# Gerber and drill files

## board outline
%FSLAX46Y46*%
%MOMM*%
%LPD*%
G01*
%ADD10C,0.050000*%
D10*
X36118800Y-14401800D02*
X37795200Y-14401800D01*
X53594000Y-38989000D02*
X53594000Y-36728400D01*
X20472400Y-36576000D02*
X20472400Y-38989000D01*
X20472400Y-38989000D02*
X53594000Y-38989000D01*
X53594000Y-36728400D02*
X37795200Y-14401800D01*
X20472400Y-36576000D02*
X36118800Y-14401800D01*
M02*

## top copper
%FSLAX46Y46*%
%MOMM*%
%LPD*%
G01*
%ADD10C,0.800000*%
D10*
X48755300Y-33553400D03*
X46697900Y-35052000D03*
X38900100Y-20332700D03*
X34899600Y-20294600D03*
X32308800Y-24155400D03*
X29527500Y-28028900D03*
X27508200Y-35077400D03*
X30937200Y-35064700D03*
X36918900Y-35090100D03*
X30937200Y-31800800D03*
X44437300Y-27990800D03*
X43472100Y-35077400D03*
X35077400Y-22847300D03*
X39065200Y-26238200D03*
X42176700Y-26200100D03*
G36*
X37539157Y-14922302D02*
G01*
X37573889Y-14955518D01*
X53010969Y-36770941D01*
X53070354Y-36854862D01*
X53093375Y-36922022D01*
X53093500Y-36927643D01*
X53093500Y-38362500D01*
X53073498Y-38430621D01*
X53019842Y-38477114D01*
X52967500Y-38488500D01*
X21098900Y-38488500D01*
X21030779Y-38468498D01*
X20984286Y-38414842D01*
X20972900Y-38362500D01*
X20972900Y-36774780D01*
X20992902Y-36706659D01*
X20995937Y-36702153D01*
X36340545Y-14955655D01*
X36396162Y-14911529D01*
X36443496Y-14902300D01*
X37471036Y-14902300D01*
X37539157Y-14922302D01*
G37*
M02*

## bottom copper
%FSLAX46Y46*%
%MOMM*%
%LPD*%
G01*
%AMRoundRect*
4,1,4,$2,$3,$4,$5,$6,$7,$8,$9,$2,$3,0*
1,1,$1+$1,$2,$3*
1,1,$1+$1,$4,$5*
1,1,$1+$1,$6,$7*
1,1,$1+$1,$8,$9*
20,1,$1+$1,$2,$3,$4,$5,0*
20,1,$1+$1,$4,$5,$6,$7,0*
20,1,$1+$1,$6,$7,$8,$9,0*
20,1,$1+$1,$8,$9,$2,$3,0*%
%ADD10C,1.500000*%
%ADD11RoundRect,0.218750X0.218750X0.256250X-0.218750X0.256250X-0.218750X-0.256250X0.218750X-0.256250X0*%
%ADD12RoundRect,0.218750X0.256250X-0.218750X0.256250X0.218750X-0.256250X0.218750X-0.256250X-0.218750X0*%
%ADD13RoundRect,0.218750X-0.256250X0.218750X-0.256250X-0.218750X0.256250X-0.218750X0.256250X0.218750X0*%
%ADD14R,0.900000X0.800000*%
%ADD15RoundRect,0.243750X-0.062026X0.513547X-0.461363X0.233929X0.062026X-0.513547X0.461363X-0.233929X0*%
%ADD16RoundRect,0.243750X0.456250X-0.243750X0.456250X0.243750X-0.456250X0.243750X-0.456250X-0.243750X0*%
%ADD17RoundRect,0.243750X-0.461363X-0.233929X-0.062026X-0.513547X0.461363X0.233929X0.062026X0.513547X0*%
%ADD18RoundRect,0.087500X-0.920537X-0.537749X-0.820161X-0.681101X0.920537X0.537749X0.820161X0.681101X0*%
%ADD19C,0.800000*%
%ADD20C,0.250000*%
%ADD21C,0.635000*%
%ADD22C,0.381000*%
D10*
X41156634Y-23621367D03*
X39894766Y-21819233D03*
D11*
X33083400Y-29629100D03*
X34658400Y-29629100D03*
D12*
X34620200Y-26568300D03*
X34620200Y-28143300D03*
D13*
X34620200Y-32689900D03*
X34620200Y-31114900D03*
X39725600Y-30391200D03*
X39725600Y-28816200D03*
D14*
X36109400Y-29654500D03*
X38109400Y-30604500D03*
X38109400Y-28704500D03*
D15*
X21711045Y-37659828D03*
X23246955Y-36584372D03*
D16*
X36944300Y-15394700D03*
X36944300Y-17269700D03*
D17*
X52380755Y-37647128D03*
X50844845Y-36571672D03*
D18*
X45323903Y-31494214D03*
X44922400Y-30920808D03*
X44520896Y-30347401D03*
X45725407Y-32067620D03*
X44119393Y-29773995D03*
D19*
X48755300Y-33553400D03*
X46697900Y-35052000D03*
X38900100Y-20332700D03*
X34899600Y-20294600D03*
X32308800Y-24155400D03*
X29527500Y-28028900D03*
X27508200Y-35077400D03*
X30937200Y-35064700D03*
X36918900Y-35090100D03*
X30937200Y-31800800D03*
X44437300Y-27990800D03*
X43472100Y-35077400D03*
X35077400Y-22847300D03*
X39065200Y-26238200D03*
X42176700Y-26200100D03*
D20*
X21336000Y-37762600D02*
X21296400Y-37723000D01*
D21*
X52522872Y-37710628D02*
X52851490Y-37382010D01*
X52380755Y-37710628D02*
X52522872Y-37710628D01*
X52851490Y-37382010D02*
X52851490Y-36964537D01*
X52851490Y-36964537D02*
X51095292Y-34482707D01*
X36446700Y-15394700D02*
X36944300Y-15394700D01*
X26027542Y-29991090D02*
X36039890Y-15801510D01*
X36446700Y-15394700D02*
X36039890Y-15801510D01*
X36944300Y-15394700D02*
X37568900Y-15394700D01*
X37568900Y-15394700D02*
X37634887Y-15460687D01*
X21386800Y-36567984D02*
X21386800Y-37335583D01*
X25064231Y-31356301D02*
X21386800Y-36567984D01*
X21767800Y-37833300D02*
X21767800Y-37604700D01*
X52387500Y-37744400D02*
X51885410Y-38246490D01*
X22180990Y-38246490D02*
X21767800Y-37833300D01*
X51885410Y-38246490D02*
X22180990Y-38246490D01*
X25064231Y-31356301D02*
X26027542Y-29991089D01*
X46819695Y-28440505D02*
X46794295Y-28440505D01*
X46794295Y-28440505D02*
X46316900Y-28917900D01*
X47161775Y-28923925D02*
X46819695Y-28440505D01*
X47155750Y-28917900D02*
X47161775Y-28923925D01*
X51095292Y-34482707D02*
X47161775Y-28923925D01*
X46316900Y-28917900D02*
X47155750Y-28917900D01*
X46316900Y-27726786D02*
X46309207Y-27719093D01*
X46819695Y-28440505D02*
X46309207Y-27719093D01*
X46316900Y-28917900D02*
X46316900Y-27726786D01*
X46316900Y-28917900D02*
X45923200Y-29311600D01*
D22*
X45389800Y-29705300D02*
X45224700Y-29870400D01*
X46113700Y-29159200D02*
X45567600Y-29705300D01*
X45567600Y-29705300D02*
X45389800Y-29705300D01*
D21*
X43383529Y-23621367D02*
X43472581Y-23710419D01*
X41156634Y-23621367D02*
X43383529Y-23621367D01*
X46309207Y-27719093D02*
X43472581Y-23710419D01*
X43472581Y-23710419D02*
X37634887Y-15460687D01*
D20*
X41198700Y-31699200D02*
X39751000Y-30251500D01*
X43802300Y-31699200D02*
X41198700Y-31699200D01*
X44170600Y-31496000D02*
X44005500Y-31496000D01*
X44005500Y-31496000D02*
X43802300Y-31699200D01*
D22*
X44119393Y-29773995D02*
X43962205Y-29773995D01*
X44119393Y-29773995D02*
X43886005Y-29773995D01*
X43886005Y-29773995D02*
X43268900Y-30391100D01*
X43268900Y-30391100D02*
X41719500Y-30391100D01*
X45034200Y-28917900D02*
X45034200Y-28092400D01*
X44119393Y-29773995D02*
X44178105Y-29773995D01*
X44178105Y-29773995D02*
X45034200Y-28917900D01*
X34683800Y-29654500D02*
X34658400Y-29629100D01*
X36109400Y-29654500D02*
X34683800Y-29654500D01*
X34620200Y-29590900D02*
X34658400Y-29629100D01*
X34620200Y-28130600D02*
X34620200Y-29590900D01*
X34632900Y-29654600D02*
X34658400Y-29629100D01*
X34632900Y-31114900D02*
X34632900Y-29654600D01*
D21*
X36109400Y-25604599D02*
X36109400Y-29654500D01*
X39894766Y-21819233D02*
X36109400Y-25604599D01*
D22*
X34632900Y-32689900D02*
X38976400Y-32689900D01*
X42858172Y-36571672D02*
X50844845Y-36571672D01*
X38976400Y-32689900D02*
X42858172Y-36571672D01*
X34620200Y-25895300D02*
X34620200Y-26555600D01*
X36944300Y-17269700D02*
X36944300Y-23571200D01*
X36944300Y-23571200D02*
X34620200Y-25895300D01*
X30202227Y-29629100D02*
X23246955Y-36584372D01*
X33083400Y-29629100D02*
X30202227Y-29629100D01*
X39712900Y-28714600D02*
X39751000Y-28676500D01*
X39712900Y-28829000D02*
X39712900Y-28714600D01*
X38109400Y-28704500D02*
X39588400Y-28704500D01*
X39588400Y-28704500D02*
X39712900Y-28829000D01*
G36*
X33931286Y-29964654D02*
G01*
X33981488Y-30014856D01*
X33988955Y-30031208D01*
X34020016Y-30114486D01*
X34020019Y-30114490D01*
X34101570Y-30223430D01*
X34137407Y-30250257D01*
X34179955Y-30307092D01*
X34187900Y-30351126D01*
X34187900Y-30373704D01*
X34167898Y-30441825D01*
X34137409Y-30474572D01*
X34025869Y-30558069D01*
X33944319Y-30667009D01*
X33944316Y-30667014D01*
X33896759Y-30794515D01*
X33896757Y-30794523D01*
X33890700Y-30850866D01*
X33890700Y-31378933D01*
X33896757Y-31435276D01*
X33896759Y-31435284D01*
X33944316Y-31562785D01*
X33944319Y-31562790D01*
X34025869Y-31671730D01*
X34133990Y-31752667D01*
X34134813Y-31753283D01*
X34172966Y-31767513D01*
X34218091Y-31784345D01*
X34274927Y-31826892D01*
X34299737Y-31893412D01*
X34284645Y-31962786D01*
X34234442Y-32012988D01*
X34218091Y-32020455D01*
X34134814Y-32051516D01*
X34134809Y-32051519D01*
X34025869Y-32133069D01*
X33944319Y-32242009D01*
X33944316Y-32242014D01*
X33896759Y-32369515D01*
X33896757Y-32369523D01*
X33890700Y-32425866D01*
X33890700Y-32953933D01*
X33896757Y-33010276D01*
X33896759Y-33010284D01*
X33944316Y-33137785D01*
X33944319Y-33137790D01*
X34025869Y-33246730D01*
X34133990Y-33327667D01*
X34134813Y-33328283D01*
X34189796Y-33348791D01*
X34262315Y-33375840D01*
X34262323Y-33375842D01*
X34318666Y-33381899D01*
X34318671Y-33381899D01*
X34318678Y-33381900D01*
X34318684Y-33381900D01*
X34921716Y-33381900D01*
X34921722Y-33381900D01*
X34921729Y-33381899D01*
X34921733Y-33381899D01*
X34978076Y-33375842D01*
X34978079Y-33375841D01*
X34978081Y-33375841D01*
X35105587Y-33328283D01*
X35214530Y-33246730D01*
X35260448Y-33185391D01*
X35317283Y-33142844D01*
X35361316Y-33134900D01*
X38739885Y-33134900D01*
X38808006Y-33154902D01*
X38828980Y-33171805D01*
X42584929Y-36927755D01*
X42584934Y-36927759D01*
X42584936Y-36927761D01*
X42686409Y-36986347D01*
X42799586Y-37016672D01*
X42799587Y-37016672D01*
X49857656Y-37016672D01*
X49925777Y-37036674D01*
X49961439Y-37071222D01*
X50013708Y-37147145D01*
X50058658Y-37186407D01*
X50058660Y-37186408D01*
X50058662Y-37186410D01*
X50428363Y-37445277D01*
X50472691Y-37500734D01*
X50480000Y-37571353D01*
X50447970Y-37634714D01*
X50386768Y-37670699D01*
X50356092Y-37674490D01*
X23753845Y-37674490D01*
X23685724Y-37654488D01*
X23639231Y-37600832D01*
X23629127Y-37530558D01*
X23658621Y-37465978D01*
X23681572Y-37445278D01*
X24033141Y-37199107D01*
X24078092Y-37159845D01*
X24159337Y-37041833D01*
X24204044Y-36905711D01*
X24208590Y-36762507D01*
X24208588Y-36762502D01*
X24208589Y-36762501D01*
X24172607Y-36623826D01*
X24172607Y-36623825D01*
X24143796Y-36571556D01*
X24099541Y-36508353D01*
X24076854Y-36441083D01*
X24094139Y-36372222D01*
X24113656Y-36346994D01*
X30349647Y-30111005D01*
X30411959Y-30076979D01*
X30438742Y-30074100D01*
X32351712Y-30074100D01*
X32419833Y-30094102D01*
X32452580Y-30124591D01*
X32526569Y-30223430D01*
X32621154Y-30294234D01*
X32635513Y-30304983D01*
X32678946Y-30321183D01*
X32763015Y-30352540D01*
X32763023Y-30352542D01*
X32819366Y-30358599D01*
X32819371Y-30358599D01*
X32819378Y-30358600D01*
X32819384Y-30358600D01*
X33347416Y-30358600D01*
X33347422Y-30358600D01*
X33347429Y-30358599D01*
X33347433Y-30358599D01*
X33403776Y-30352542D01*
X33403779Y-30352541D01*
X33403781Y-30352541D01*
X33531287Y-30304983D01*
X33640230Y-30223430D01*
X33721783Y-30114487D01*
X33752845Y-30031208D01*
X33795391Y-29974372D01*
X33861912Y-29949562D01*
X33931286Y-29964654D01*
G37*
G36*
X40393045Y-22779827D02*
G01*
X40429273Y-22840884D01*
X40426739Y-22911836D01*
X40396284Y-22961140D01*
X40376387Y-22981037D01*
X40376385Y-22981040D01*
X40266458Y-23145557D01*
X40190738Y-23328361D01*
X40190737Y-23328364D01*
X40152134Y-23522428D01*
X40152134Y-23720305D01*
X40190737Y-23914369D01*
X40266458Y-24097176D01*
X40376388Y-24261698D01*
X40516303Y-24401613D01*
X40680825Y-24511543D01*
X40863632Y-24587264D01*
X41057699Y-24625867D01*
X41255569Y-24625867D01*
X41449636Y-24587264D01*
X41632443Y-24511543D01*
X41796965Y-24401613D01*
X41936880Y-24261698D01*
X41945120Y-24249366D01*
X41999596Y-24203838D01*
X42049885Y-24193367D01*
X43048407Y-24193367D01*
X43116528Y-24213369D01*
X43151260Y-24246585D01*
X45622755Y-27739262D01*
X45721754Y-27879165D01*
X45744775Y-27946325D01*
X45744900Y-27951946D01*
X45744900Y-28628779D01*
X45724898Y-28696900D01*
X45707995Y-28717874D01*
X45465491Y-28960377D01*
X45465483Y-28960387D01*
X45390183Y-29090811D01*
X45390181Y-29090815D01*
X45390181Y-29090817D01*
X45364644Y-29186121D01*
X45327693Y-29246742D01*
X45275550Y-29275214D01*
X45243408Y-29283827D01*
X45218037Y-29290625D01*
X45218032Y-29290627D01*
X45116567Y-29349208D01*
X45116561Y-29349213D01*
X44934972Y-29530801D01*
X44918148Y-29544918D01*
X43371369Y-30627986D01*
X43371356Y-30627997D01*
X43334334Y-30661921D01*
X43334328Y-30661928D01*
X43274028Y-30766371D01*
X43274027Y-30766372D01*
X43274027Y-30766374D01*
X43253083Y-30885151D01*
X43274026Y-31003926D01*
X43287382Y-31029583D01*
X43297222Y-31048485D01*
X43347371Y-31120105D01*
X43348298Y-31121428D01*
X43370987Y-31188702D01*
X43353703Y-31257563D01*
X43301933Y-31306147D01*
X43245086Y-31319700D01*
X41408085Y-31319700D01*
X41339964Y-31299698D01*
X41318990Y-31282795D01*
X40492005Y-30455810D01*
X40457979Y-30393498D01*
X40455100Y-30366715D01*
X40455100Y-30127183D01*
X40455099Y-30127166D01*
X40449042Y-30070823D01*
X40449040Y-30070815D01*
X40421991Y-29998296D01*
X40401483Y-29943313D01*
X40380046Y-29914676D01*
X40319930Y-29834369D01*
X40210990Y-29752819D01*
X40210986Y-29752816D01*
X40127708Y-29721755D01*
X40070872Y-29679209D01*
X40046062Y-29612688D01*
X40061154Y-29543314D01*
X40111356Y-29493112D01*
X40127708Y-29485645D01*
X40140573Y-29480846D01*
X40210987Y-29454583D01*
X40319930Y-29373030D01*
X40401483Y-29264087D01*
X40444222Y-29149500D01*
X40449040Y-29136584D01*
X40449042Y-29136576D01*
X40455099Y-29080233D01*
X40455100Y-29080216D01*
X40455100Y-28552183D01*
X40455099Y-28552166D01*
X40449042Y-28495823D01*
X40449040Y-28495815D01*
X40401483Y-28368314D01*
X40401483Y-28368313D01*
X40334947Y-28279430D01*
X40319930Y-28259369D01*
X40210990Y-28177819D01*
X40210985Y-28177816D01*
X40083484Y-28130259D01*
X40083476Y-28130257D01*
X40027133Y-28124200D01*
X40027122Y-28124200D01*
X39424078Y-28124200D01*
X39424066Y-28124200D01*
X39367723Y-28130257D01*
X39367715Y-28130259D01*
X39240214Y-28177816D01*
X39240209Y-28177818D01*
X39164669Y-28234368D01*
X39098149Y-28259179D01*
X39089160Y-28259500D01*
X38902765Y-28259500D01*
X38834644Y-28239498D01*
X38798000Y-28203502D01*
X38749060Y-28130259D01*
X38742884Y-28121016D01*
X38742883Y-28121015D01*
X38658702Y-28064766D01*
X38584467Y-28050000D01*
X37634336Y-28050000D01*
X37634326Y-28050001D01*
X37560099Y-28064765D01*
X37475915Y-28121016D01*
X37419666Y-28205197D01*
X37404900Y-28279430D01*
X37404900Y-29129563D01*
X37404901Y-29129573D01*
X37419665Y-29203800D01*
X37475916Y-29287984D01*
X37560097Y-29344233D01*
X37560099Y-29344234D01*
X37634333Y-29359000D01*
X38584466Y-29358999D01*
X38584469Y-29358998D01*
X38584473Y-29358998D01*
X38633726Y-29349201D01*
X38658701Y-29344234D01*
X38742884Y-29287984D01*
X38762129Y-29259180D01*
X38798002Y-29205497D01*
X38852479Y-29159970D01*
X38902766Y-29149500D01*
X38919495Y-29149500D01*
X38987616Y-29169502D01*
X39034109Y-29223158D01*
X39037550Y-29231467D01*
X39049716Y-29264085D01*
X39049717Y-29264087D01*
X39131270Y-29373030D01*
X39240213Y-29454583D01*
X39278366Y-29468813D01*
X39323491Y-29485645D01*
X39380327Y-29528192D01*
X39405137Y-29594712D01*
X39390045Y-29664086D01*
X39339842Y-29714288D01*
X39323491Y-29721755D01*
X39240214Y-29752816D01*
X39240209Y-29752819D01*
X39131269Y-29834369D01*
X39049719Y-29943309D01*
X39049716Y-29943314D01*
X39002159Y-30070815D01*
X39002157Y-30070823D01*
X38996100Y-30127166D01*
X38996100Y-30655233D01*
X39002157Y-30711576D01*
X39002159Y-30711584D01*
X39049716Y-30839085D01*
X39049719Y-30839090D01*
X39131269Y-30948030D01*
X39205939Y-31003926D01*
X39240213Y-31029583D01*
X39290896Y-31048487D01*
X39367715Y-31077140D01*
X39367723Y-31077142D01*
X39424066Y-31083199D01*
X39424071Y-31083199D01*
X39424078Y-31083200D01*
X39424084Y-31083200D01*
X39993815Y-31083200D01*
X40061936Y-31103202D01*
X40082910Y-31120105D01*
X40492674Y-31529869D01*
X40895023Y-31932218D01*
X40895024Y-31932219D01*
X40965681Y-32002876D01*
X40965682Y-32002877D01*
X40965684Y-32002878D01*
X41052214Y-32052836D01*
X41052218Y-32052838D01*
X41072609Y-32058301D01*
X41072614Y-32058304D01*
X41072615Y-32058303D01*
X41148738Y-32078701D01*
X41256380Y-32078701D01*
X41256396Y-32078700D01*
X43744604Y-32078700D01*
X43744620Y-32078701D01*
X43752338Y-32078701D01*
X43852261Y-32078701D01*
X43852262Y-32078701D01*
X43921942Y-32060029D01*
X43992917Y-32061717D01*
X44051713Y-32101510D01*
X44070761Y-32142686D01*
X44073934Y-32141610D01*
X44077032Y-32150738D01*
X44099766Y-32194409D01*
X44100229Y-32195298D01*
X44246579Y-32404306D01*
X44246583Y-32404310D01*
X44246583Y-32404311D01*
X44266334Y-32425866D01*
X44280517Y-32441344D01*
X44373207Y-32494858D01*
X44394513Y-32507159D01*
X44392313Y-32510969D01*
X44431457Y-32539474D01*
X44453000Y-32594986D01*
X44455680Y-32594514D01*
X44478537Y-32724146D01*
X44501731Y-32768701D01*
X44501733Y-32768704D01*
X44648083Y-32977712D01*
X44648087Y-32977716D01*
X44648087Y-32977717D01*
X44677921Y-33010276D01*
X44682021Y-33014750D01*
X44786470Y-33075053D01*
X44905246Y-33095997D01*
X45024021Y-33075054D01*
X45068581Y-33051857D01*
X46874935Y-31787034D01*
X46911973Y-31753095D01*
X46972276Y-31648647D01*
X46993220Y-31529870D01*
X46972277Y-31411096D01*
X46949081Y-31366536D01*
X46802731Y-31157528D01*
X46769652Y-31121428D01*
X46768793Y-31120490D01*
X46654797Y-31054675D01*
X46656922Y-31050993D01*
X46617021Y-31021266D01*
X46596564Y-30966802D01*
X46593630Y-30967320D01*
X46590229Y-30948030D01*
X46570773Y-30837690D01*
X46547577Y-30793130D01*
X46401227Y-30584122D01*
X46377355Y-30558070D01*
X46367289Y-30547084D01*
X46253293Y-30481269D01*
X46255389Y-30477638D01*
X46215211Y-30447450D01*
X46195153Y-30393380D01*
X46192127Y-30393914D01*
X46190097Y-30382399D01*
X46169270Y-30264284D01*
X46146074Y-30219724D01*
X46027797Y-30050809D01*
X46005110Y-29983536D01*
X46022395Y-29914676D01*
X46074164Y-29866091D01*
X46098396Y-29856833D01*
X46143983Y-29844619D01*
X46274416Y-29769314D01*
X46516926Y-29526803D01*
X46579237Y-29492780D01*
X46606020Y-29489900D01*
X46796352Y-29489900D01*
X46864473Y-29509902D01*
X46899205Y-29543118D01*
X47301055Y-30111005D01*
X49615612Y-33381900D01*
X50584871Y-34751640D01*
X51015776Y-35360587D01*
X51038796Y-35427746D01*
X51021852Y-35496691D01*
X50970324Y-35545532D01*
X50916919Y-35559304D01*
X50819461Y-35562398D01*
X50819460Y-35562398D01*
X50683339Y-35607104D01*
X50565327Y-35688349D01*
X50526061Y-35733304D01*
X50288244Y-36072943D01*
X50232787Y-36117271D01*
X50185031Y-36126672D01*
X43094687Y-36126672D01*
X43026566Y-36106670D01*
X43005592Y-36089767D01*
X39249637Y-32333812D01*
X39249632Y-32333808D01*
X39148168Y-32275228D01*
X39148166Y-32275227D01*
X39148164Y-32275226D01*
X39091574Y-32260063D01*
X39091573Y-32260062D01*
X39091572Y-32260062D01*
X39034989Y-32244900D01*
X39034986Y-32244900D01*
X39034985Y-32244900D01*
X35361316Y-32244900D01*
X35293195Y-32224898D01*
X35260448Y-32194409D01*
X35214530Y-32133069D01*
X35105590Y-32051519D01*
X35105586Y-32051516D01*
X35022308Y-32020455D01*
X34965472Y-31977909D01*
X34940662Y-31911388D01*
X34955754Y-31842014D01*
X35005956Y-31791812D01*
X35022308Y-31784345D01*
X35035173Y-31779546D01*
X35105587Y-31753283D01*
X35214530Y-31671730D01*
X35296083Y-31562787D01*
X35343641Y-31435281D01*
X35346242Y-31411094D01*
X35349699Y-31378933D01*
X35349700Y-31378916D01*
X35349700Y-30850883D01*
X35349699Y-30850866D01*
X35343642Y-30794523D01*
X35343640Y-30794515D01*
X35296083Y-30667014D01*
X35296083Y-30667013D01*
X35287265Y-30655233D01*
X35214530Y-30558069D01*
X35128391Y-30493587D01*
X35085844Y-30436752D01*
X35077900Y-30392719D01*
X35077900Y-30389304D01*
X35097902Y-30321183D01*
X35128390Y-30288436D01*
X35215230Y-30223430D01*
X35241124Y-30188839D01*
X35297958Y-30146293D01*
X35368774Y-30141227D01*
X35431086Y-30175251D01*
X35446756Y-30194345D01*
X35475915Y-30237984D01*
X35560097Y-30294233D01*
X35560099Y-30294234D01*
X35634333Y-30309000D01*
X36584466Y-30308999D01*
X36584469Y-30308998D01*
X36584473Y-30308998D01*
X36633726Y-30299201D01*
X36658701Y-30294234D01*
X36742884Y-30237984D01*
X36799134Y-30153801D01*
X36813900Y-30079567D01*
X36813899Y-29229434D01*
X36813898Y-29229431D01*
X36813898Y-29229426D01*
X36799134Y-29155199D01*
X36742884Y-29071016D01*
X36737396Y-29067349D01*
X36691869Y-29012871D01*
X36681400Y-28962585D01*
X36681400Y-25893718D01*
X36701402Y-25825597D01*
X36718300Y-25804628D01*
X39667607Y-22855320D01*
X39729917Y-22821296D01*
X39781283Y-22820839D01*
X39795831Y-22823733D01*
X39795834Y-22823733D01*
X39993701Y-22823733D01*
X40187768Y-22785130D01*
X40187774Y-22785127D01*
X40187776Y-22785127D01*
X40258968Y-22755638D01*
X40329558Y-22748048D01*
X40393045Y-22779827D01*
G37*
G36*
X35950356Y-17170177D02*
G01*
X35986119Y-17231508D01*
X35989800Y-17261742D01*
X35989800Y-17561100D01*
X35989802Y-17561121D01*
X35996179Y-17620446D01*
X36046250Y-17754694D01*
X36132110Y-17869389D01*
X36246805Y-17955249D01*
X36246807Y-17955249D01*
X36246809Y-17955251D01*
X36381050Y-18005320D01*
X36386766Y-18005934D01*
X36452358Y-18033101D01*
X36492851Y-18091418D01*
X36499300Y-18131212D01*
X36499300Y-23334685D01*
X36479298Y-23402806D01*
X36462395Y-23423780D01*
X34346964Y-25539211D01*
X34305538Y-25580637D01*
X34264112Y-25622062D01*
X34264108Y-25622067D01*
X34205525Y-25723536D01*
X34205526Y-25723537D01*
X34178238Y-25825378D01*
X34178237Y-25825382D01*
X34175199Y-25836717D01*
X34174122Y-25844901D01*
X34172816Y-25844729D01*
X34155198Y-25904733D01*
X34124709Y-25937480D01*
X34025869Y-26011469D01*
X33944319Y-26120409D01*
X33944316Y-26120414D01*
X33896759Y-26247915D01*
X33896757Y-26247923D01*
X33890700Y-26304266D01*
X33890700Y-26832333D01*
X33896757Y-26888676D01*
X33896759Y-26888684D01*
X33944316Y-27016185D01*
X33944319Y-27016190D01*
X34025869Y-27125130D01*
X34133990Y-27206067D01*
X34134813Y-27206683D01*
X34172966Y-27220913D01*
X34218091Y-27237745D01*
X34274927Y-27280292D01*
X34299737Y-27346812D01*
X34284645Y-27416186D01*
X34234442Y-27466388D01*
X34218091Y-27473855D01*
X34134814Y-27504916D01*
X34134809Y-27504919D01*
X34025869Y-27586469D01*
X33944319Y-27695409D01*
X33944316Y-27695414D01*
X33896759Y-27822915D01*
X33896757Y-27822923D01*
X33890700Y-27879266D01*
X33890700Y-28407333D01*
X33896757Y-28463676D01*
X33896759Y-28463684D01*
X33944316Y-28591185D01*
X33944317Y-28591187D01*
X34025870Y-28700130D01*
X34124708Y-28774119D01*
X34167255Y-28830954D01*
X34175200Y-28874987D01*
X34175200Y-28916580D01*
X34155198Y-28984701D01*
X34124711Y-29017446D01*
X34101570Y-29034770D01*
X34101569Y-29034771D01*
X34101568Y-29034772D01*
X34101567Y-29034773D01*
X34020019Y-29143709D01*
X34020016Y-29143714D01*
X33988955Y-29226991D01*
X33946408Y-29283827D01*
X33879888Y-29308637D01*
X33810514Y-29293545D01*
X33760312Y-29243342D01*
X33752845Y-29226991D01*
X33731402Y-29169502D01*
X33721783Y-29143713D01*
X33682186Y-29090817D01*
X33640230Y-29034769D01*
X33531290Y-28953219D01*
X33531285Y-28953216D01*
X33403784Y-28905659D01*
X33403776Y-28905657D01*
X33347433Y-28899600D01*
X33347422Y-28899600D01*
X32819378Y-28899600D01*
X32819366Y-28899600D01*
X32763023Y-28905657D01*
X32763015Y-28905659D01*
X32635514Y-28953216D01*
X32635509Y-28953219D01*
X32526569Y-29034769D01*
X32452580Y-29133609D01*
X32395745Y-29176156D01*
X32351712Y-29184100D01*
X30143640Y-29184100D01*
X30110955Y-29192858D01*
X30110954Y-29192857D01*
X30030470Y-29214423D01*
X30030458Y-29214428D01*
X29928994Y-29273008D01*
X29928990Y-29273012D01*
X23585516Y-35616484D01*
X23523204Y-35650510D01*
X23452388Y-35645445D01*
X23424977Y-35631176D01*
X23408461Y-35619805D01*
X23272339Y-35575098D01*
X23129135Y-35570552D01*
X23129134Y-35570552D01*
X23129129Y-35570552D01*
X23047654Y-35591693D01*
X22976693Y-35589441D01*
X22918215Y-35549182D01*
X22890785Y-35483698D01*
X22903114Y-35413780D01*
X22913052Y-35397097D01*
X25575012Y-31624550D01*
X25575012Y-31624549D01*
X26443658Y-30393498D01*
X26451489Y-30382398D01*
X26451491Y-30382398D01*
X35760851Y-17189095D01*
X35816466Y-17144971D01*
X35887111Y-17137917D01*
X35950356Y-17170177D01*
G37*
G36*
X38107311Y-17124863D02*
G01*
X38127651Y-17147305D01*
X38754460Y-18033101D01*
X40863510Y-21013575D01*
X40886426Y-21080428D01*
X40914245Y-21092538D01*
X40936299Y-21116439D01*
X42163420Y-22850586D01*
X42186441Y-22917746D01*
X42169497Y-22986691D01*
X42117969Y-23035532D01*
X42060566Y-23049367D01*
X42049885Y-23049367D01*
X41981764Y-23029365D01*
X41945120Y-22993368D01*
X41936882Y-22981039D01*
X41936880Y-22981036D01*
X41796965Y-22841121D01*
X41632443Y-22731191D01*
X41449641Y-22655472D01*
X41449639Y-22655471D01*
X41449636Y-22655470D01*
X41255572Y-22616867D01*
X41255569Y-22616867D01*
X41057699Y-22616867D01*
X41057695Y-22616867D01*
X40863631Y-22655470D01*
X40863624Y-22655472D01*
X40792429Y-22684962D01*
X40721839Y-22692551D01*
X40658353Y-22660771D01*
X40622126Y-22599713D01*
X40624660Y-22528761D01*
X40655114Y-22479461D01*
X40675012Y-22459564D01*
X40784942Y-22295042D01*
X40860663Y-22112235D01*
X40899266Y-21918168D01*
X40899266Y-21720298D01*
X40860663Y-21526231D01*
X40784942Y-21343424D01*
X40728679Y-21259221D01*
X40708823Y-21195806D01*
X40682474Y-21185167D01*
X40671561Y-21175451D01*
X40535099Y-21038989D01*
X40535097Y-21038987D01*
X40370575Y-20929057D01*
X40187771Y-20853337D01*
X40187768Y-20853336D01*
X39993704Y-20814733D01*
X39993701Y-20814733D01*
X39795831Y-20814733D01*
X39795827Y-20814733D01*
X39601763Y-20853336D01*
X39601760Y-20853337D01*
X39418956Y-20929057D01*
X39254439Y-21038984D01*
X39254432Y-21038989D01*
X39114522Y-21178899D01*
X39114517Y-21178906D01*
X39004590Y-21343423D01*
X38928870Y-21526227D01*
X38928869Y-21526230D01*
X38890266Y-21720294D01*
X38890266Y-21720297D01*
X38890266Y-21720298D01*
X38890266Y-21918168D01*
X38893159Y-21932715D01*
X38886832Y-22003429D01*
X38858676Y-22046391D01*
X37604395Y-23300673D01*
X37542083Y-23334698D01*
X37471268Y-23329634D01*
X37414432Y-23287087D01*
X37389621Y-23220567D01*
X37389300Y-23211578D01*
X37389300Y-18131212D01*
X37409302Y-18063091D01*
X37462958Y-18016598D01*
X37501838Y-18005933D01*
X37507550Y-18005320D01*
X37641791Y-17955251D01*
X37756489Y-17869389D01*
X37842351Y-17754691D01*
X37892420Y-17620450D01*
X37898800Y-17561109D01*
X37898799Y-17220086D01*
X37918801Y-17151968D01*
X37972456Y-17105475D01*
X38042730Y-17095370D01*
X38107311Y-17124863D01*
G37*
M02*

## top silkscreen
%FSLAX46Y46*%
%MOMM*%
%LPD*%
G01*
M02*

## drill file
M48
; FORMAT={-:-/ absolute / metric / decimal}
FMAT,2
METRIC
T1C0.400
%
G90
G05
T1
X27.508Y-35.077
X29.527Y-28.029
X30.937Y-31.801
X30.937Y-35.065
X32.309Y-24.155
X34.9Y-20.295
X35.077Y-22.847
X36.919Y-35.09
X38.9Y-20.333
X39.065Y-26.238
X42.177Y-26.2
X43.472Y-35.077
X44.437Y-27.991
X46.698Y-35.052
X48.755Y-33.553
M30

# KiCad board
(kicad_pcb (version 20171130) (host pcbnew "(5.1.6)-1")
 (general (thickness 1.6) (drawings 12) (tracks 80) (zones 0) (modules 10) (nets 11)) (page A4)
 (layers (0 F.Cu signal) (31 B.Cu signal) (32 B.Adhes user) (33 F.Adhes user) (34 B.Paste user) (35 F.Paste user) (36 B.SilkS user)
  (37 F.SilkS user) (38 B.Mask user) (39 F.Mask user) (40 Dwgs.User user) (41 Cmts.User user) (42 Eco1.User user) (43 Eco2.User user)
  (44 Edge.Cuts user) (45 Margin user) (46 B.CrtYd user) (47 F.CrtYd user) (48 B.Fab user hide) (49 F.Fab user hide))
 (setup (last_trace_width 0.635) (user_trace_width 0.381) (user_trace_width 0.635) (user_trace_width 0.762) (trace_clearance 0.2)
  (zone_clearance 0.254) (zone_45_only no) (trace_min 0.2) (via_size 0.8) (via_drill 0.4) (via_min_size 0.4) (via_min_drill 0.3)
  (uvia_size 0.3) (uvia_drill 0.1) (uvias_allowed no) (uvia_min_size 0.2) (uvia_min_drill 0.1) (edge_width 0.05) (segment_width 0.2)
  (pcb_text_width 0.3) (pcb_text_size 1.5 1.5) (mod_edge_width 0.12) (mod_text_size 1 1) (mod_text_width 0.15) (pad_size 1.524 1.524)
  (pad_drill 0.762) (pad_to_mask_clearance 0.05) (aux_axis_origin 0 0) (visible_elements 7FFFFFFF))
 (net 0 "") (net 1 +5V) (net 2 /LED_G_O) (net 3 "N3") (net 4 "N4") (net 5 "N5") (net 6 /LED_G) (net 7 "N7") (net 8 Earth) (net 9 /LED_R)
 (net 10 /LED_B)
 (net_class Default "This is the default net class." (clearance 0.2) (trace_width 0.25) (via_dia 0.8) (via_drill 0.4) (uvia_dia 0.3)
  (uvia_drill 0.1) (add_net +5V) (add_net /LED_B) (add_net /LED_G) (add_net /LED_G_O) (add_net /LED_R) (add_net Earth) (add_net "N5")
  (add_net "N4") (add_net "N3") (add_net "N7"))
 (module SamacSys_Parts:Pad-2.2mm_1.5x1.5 (layer B.Cu) (at 40.5257 22.7203 125)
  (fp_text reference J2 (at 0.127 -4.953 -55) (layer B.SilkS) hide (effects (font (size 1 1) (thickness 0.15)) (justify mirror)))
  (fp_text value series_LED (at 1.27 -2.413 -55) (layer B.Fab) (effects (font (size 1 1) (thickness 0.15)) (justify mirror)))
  (pad 1 smd circle (at -1.1 0 125) (size 1.5 1.5) (layers B.Cu B.Paste B.Mask) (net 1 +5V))
  (pad 2 smd circle (at 1.1 0 125) (size 1.5 1.5) (layers B.Cu B.Paste B.Mask) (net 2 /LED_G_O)))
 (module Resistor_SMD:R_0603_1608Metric (layer B.Cu) (at 33.8709 29.6291 180)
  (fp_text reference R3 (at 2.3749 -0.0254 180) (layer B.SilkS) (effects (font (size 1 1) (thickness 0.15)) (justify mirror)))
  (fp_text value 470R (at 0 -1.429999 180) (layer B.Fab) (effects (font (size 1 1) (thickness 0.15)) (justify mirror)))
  (pad 2 smd roundrect (at 0.7875 0 180) (size 0.875 0.95) (layers B.Cu B.Paste B.Mask) (roundrect_rratio 0.25) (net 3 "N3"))
  (pad 1 smd roundrect (at -0.7875 0 180) (size 0.875 0.95) (layers B.Cu B.Paste B.Mask) (roundrect_rratio 0.25) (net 2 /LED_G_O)))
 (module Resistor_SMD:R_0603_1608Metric (layer B.Cu) (at 34.6202 27.3558 90)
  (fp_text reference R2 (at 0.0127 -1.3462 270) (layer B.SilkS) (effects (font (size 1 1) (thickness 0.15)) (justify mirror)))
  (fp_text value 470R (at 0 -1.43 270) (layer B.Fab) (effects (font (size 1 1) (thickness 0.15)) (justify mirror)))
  (pad 2 smd roundrect (at 0.7875 0 90) (size 0.875 0.95) (layers B.Cu B.Paste B.Mask) (roundrect_rratio 0.25) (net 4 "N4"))
  (pad 1 smd roundrect (at -0.7875 0 90) (size 0.875 0.95) (layers B.Cu B.Paste B.Mask) (roundrect_rratio 0.25) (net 2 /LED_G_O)))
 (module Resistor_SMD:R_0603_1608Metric (layer B.Cu) (at 34.6202 31.9024 270)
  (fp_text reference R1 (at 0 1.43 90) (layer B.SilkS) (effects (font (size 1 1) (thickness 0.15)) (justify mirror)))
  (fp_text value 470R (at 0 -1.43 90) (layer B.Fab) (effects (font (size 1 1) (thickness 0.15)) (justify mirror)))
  (pad 2 smd roundrect (at 0.7875 0 270) (size 0.875 0.95) (layers B.Cu B.Paste B.Mask) (roundrect_rratio 0.25) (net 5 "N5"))
  (pad 1 smd roundrect (at -0.7875 0 270) (size 0.875 0.95) (layers B.Cu B.Paste B.Mask) (roundrect_rratio 0.25) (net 2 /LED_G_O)))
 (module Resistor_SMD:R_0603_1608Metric (layer B.Cu) (at 39.7256 29.6037 270)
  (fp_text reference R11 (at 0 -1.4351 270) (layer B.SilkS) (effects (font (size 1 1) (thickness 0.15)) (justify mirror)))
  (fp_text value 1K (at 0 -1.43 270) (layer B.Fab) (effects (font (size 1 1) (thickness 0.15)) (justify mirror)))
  (pad 2 smd roundrect (at 0.7875 0 270) (size 0.875 0.95) (layers B.Cu B.Paste B.Mask) (roundrect_rratio 0.25) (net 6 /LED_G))
  (pad 1 smd roundrect (at -0.7875 0 270) (size 0.875 0.95) (layers B.Cu B.Paste B.Mask) (roundrect_rratio 0.25) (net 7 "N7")))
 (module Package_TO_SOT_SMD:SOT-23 (layer B.Cu) (at 37.1094 29.6545 180)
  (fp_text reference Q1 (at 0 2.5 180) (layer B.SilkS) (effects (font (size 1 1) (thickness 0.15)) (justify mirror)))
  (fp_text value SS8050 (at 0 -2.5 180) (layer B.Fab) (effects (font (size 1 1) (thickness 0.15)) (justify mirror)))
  (pad 3 smd rect (at 1 0 180) (size 0.9 0.8) (layers B.Cu B.Paste B.Mask) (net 2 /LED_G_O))
  (pad 2 smd rect (at -1 -0.95 180) (size 0.9 0.8) (layers B.Cu B.Paste B.Mask) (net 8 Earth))
  (pad 1 smd rect (at -1 0.95 180) (size 0.9 0.8) (layers B.Cu B.Paste B.Mask) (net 7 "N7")))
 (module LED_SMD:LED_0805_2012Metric (layer B.Cu) (at 22.479 37.1221 215)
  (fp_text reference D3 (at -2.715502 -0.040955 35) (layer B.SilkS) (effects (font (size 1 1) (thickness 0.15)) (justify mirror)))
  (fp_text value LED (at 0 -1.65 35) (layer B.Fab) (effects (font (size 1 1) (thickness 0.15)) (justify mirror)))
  (pad 2 smd roundrect (at 0.9375 0 215) (size 0.975 1.4) (layers B.Cu B.Paste B.Mask) (roundrect_rratio 0.25) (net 1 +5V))
  (pad 1 smd roundrect (at -0.9375 0 215) (size 0.975 1.4) (layers B.Cu B.Paste B.Mask) (roundrect_rratio 0.25) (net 3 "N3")))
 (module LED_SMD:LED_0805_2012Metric (layer B.Cu) (at 36.9443 16.3322 90)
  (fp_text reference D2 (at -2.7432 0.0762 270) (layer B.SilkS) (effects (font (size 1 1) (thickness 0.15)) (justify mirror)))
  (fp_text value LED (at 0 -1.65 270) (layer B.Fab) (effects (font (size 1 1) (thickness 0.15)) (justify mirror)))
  (pad 2 smd roundrect (at 0.9375 0 90) (size 0.975 1.4) (layers B.Cu B.Paste B.Mask) (roundrect_rratio 0.25) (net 1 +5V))
  (pad 1 smd roundrect (at -0.9375 0 90) (size 0.975 1.4) (layers B.Cu B.Paste B.Mask) (roundrect_rratio 0.25) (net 4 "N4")))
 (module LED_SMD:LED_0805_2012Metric (layer B.Cu) (at 51.6128 37.1094 325)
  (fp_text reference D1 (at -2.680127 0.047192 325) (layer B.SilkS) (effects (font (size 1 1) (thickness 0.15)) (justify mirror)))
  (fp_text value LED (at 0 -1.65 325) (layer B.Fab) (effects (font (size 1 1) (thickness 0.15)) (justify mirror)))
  (pad 2 smd roundrect (at 0.9375 0 325) (size 0.975 1.4) (layers B.Cu B.Paste B.Mask) (roundrect_rratio 0.25) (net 1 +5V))
  (pad 1 smd roundrect (at -0.9375 0 325) (size 0.975 1.4) (layers B.Cu B.Paste B.Mask) (roundrect_rratio 0.25) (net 5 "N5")))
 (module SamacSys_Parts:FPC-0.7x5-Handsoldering (layer B.Cu) (at 44.9072 30.8991 305)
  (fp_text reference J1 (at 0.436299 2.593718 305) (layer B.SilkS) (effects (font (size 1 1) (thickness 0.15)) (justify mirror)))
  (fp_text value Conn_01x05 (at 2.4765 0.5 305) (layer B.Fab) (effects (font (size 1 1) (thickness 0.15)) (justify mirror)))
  (pad 4 smd roundrect (at 0.7265 0 305) (size 0.35 2.3) (layers B.Cu B.Paste B.Mask) (roundrect_rratio 0.25) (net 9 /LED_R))
  (pad 3 smd roundrect (at 0.0265 0 305) (size 0.35 2.3) (layers B.Cu B.Paste B.Mask) (roundrect_rratio 0.25) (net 6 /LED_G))
  (pad 2 smd roundrect (at -0.6735 0 305) (size 0.35 2.3) (layers B.Cu B.Paste B.Mask) (roundrect_rratio 0.25) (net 1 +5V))
  (pad 5 smd roundrect (at 1.4265 0 305) (size 0.35 2.3) (layers B.Cu B.Paste B.Mask) (roundrect_rratio 0.25) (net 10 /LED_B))
  (pad 1 smd roundrect (at -1.3735 0 305) (size 0.35 2.3) (layers B.Cu B.Paste B.Mask) (roundrect_rratio 0.25) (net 8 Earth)))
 (gr_line (start 36.1188 14.4018) (end 37.7952 14.4018) (layer Edge.Cuts) (width 0.05))
 (gr_line (start 53.594 38.989) (end 53.594 36.7284) (layer Edge.Cuts) (width 0.05))
 (gr_line (start 20.4724 36.576) (end 20.4724 38.989) (layer Edge.Cuts) (width 0.05))
 (gr_line (start 20.4724 38.989) (end 53.594 38.989) (layer Edge.Cuts) (width 0.05))
 (gr_line (start 53.594 36.7284) (end 37.7952 14.4018) (layer Edge.Cuts) (width 0.05))
 (gr_line (start 20.4724 36.576) (end 36.1188 14.4018) (layer Edge.Cuts) (width 0.05))
 (segment (start 21.336 37.7626) (end 21.2964 37.723) (width 0.25) (layer B.Cu) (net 1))
 (segment (start 52.522872 37.710628) (end 52.85149 37.38201) (width 0.635) (layer B.Cu) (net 1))
 (segment (start 52.380755 37.710628) (end 52.522872 37.710628) (width 0.635) (layer B.Cu) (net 1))
 (segment (start 52.85149 37.38201) (end 52.85149 36.964537) (width 0.635) (layer B.Cu) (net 1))
 (segment (start 52.85149 36.964537) (end 51.095292 34.482707) (width 0.635) (layer B.Cu) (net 1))
 (segment (start 36.4467 15.3947) (end 36.9443 15.3947) (width 0.635) (layer B.Cu) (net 1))
 (segment (start 26.027542 29.99109) (end 36.03989 15.80151) (width 0.635) (layer B.Cu) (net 1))
 (segment (start 36.4467 15.3947) (end 36.03989 15.80151) (width 0.635) (layer B.Cu) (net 1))
 (segment (start 36.9443 15.3947) (end 37.5689 15.3947) (width 0.635) (layer B.Cu) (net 1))
 (segment (start 37.5689 15.3947) (end 37.634887 15.460687) (width 0.635) (layer B.Cu) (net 1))
 (segment (start 21.3868 36.567984) (end 21.3868 37.335583) (width 0.635) (layer B.Cu) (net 1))
 (segment (start 25.064231 31.356301) (end 21.3868 36.567984) (width 0.635) (layer B.Cu) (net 1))
 (segment (start 21.7678 37.8333) (end 21.7678 37.6047) (width 0.635) (layer B.Cu) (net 1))
 (segment (start 52.3875 37.7444) (end 51.88541 38.24649) (width 0.635) (layer B.Cu) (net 1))
 (segment (start 22.18099 38.24649) (end 21.7678 37.8333) (width 0.635) (layer B.Cu) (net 1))
 (segment (start 51.88541 38.24649) (end 22.18099 38.24649) (width 0.635) (layer B.Cu) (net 1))
 (segment (start 25.064231 31.356301) (end 26.027542 29.991089) (width 0.635) (layer B.Cu) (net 1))
 (segment (start 46.819695 28.440505) (end 46.794295 28.440505) (width 0.635) (layer B.Cu) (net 1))
 (segment (start 46.794295 28.440505) (end 46.3169 28.9179) (width 0.635) (layer B.Cu) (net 1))
 (segment (start 47.161775 28.923925) (end 46.819695 28.440505) (width 0.635) (layer B.Cu) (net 1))
 (segment (start 47.15575 28.9179) (end 47.161775 28.923925) (width 0.635) (layer B.Cu) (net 1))
 (segment (start 51.095292 34.482707) (end 47.161775 28.923925) (width 0.635) (layer B.Cu) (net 1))
 (segment (start 46.3169 28.9179) (end 47.15575 28.9179) (width 0.635) (layer B.Cu) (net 1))
 (segment (start 46.3169 27.726786) (end 46.309207 27.719093) (width 0.635) (layer B.Cu) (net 1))
 (segment (start 46.819695 28.440505) (end 46.309207 27.719093) (width 0.635) (layer B.Cu) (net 1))
 (segment (start 46.3169 28.9179) (end 46.3169 27.726786) (width 0.635) (layer B.Cu) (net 1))
 (segment (start 46.3169 28.9179) (end 45.9232 29.3116) (width 0.635) (layer B.Cu) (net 1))
 (segment (start 45.3898 29.7053) (end 45.2247 29.8704) (width 0.381) (layer B.Cu) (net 1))
 (segment (start 46.1137 29.1592) (end 45.5676 29.7053) (width 0.381) (layer B.Cu) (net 1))
 (segment (start 45.5676 29.7053) (end 45.3898 29.7053) (width 0.381) (layer B.Cu) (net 1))
 (segment (start 43.383529 23.621367) (end 43.472581 23.710419) (width 0.635) (layer B.Cu) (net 1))
 (segment (start 41.156634 23.621367) (end 43.383529 23.621367) (width 0.635) (layer B.Cu) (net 1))
 (segment (start 46.309207 27.719093) (end 43.472581 23.710419) (width 0.635) (layer B.Cu) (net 1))
 (segment (start 43.472581 23.710419) (end 37.634887 15.460687) (width 0.635) (layer B.Cu) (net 1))
 (segment (start 41.1987 31.6992) (end 39.751 30.2515) (width 0.25) (layer B.Cu) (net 6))
 (segment (start 43.8023 31.6992) (end 41.1987 31.6992) (width 0.25) (layer B.Cu) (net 6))
 (segment (start 44.1706 31.496) (end 44.0055 31.496) (width 0.25) (layer B.Cu) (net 6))
 (segment (start 44.0055 31.496) (end 43.8023 31.6992) (width 0.25) (layer B.Cu) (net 6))
 (via (at 48.7553 33.5534) (size 0.8) (drill 0.4) (layers F.Cu B.Cu) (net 8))
 (via (at 46.6979 35.052) (size 0.8) (drill 0.4) (layers F.Cu B.Cu) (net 8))
 (via (at 38.9001 20.3327) (size 0.8) (drill 0.4) (layers F.Cu B.Cu) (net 8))
 (via (at 34.8996 20.2946) (size 0.8) (drill 0.4) (layers F.Cu B.Cu) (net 8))
 (via (at 32.3088 24.1554) (size 0.8) (drill 0.4) (layers F.Cu B.Cu) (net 8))
 (via (at 29.5275 28.0289) (size 0.8) (drill 0.4) (layers F.Cu B.Cu) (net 8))
 (via (at 27.5082 35.0774) (size 0.8) (drill 0.4) (layers F.Cu B.Cu) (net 8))
 (via (at 30.9372 35.0647) (size 0.8) (drill 0.4) (layers F.Cu B.Cu) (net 8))
 (via (at 36.9189 35.0901) (size 0.8) (drill 0.4) (layers F.Cu B.Cu) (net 8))
 (via (at 30.9372 31.8008) (size 0.8) (drill 0.4) (layers F.Cu B.Cu) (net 8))
 (segment (start 44.119393 29.773995) (end 43.962205 29.773995) (width 0.381) (layer B.Cu) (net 8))
 (segment (start 44.119393 29.773995) (end 43.886005 29.773995) (width 0.381) (layer B.Cu) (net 8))
 (segment (start 43.886005 29.773995) (end 43.2689 30.3911) (width 0.381) (layer B.Cu) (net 8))
 (segment (start 43.2689 30.3911) (end 41.7195 30.3911) (width 0.381) (layer B.Cu) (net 8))
 (segment (start 45.0342 28.9179) (end 45.0342 28.0924) (width 0.381) (layer B.Cu) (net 8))
 (segment (start 44.119393 29.773995) (end 44.178105 29.773995) (width 0.381) (layer B.Cu) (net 8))
 (segment (start 44.178105 29.773995) (end 45.0342 28.9179) (width 0.381) (layer B.Cu) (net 8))
 (via (at 44.4373 27.9908) (size 0.8) (drill 0.4) (layers F.Cu B.Cu) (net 8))
 (via (at 43.4721 35.0774) (size 0.8) (drill 0.4) (layers F.Cu B.Cu) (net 8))
 (via (at 35.0774 22.8473) (size 0.8) (drill 0.4) (layers F.Cu B.Cu) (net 8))
 (via (at 39.0652 26.2382) (size 0.8) (drill 0.4) (layers F.Cu B.Cu) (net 8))
 (via (at 42.1767 26.2001) (size 0.8) (drill 0.4) (layers F.Cu B.Cu) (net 8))
 (segment (start 34.6838 29.6545) (end 34.6584 29.6291) (width 0.381) (layer B.Cu) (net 2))
 (segment (start 36.1094 29.6545) (end 34.6838 29.6545) (width 0.381) (layer B.Cu) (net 2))
 (segment (start 34.6202 29.5909) (end 34.6584 29.6291) (width 0.381) (layer B.Cu) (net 2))
 (segment (start 34.6202 28.1306) (end 34.6202 29.5909) (width 0.381) (layer B.Cu) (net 2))
 (segment (start 34.6329 29.6546) (end 34.6584 29.6291) (width 0.381) (layer B.Cu) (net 2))
 (segment (start 34.6329 31.1149) (end 34.6329 29.6546) (width 0.381) (layer B.Cu) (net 2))
 (segment (start 36.1094 25.604599) (end 36.1094 29.6545) (width 0.635) (layer B.Cu) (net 2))
 (segment (start 39.894766 21.819233) (end 36.1094 25.604599) (width 0.635) (layer B.Cu) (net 2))
 (segment (start 34.6329 32.6899) (end 38.9764 32.6899) (width 0.381) (layer B.Cu) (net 5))
 (segment (start 42.858172 36.571672) (end 50.844845 36.571672) (width 0.381) (layer B.Cu) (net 5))
 (segment (start 38.9764 32.6899) (end 42.858172 36.571672) (width 0.381) (layer B.Cu) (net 5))
 (segment (start 34.6202 25.8953) (end 34.6202 26.5556) (width 0.381) (layer B.Cu) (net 4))
 (segment (start 36.9443 17.2697) (end 36.9443 23.5712) (width 0.381) (layer B.Cu) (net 4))
 (segment (start 36.9443 23.5712) (end 34.6202 25.8953) (width 0.381) (layer B.Cu) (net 4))
 (segment (start 30.202227 29.6291) (end 23.246955 36.584372) (width 0.381) (layer B.Cu) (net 3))
 (segment (start 33.0834 29.6291) (end 30.202227 29.6291) (width 0.381) (layer B.Cu) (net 3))
 (segment (start 39.7129 28.7146) (end 39.751 28.6765) (width 0.381) (layer B.Cu) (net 7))
 (segment (start 39.7129 28.829) (end 39.7129 28.7146) (width 0.381) (layer B.Cu) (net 7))
 (segment (start 38.1094 28.7045) (end 39.5884 28.7045) (width 0.381) (layer B.Cu) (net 7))
 (segment (start 39.5884 28.7045) (end 39.7129 28.829) (width 0.381) (layer B.Cu) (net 7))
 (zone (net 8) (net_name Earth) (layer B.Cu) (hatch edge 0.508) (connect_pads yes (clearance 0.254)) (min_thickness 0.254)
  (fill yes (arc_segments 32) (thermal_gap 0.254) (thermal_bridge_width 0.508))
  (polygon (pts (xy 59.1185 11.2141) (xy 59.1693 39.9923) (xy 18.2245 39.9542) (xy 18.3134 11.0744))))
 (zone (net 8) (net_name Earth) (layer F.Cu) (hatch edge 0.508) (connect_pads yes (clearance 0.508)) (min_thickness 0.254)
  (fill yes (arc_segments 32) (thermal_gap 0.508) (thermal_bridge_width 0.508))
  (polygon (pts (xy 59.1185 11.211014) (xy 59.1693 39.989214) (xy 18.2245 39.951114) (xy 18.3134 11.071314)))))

